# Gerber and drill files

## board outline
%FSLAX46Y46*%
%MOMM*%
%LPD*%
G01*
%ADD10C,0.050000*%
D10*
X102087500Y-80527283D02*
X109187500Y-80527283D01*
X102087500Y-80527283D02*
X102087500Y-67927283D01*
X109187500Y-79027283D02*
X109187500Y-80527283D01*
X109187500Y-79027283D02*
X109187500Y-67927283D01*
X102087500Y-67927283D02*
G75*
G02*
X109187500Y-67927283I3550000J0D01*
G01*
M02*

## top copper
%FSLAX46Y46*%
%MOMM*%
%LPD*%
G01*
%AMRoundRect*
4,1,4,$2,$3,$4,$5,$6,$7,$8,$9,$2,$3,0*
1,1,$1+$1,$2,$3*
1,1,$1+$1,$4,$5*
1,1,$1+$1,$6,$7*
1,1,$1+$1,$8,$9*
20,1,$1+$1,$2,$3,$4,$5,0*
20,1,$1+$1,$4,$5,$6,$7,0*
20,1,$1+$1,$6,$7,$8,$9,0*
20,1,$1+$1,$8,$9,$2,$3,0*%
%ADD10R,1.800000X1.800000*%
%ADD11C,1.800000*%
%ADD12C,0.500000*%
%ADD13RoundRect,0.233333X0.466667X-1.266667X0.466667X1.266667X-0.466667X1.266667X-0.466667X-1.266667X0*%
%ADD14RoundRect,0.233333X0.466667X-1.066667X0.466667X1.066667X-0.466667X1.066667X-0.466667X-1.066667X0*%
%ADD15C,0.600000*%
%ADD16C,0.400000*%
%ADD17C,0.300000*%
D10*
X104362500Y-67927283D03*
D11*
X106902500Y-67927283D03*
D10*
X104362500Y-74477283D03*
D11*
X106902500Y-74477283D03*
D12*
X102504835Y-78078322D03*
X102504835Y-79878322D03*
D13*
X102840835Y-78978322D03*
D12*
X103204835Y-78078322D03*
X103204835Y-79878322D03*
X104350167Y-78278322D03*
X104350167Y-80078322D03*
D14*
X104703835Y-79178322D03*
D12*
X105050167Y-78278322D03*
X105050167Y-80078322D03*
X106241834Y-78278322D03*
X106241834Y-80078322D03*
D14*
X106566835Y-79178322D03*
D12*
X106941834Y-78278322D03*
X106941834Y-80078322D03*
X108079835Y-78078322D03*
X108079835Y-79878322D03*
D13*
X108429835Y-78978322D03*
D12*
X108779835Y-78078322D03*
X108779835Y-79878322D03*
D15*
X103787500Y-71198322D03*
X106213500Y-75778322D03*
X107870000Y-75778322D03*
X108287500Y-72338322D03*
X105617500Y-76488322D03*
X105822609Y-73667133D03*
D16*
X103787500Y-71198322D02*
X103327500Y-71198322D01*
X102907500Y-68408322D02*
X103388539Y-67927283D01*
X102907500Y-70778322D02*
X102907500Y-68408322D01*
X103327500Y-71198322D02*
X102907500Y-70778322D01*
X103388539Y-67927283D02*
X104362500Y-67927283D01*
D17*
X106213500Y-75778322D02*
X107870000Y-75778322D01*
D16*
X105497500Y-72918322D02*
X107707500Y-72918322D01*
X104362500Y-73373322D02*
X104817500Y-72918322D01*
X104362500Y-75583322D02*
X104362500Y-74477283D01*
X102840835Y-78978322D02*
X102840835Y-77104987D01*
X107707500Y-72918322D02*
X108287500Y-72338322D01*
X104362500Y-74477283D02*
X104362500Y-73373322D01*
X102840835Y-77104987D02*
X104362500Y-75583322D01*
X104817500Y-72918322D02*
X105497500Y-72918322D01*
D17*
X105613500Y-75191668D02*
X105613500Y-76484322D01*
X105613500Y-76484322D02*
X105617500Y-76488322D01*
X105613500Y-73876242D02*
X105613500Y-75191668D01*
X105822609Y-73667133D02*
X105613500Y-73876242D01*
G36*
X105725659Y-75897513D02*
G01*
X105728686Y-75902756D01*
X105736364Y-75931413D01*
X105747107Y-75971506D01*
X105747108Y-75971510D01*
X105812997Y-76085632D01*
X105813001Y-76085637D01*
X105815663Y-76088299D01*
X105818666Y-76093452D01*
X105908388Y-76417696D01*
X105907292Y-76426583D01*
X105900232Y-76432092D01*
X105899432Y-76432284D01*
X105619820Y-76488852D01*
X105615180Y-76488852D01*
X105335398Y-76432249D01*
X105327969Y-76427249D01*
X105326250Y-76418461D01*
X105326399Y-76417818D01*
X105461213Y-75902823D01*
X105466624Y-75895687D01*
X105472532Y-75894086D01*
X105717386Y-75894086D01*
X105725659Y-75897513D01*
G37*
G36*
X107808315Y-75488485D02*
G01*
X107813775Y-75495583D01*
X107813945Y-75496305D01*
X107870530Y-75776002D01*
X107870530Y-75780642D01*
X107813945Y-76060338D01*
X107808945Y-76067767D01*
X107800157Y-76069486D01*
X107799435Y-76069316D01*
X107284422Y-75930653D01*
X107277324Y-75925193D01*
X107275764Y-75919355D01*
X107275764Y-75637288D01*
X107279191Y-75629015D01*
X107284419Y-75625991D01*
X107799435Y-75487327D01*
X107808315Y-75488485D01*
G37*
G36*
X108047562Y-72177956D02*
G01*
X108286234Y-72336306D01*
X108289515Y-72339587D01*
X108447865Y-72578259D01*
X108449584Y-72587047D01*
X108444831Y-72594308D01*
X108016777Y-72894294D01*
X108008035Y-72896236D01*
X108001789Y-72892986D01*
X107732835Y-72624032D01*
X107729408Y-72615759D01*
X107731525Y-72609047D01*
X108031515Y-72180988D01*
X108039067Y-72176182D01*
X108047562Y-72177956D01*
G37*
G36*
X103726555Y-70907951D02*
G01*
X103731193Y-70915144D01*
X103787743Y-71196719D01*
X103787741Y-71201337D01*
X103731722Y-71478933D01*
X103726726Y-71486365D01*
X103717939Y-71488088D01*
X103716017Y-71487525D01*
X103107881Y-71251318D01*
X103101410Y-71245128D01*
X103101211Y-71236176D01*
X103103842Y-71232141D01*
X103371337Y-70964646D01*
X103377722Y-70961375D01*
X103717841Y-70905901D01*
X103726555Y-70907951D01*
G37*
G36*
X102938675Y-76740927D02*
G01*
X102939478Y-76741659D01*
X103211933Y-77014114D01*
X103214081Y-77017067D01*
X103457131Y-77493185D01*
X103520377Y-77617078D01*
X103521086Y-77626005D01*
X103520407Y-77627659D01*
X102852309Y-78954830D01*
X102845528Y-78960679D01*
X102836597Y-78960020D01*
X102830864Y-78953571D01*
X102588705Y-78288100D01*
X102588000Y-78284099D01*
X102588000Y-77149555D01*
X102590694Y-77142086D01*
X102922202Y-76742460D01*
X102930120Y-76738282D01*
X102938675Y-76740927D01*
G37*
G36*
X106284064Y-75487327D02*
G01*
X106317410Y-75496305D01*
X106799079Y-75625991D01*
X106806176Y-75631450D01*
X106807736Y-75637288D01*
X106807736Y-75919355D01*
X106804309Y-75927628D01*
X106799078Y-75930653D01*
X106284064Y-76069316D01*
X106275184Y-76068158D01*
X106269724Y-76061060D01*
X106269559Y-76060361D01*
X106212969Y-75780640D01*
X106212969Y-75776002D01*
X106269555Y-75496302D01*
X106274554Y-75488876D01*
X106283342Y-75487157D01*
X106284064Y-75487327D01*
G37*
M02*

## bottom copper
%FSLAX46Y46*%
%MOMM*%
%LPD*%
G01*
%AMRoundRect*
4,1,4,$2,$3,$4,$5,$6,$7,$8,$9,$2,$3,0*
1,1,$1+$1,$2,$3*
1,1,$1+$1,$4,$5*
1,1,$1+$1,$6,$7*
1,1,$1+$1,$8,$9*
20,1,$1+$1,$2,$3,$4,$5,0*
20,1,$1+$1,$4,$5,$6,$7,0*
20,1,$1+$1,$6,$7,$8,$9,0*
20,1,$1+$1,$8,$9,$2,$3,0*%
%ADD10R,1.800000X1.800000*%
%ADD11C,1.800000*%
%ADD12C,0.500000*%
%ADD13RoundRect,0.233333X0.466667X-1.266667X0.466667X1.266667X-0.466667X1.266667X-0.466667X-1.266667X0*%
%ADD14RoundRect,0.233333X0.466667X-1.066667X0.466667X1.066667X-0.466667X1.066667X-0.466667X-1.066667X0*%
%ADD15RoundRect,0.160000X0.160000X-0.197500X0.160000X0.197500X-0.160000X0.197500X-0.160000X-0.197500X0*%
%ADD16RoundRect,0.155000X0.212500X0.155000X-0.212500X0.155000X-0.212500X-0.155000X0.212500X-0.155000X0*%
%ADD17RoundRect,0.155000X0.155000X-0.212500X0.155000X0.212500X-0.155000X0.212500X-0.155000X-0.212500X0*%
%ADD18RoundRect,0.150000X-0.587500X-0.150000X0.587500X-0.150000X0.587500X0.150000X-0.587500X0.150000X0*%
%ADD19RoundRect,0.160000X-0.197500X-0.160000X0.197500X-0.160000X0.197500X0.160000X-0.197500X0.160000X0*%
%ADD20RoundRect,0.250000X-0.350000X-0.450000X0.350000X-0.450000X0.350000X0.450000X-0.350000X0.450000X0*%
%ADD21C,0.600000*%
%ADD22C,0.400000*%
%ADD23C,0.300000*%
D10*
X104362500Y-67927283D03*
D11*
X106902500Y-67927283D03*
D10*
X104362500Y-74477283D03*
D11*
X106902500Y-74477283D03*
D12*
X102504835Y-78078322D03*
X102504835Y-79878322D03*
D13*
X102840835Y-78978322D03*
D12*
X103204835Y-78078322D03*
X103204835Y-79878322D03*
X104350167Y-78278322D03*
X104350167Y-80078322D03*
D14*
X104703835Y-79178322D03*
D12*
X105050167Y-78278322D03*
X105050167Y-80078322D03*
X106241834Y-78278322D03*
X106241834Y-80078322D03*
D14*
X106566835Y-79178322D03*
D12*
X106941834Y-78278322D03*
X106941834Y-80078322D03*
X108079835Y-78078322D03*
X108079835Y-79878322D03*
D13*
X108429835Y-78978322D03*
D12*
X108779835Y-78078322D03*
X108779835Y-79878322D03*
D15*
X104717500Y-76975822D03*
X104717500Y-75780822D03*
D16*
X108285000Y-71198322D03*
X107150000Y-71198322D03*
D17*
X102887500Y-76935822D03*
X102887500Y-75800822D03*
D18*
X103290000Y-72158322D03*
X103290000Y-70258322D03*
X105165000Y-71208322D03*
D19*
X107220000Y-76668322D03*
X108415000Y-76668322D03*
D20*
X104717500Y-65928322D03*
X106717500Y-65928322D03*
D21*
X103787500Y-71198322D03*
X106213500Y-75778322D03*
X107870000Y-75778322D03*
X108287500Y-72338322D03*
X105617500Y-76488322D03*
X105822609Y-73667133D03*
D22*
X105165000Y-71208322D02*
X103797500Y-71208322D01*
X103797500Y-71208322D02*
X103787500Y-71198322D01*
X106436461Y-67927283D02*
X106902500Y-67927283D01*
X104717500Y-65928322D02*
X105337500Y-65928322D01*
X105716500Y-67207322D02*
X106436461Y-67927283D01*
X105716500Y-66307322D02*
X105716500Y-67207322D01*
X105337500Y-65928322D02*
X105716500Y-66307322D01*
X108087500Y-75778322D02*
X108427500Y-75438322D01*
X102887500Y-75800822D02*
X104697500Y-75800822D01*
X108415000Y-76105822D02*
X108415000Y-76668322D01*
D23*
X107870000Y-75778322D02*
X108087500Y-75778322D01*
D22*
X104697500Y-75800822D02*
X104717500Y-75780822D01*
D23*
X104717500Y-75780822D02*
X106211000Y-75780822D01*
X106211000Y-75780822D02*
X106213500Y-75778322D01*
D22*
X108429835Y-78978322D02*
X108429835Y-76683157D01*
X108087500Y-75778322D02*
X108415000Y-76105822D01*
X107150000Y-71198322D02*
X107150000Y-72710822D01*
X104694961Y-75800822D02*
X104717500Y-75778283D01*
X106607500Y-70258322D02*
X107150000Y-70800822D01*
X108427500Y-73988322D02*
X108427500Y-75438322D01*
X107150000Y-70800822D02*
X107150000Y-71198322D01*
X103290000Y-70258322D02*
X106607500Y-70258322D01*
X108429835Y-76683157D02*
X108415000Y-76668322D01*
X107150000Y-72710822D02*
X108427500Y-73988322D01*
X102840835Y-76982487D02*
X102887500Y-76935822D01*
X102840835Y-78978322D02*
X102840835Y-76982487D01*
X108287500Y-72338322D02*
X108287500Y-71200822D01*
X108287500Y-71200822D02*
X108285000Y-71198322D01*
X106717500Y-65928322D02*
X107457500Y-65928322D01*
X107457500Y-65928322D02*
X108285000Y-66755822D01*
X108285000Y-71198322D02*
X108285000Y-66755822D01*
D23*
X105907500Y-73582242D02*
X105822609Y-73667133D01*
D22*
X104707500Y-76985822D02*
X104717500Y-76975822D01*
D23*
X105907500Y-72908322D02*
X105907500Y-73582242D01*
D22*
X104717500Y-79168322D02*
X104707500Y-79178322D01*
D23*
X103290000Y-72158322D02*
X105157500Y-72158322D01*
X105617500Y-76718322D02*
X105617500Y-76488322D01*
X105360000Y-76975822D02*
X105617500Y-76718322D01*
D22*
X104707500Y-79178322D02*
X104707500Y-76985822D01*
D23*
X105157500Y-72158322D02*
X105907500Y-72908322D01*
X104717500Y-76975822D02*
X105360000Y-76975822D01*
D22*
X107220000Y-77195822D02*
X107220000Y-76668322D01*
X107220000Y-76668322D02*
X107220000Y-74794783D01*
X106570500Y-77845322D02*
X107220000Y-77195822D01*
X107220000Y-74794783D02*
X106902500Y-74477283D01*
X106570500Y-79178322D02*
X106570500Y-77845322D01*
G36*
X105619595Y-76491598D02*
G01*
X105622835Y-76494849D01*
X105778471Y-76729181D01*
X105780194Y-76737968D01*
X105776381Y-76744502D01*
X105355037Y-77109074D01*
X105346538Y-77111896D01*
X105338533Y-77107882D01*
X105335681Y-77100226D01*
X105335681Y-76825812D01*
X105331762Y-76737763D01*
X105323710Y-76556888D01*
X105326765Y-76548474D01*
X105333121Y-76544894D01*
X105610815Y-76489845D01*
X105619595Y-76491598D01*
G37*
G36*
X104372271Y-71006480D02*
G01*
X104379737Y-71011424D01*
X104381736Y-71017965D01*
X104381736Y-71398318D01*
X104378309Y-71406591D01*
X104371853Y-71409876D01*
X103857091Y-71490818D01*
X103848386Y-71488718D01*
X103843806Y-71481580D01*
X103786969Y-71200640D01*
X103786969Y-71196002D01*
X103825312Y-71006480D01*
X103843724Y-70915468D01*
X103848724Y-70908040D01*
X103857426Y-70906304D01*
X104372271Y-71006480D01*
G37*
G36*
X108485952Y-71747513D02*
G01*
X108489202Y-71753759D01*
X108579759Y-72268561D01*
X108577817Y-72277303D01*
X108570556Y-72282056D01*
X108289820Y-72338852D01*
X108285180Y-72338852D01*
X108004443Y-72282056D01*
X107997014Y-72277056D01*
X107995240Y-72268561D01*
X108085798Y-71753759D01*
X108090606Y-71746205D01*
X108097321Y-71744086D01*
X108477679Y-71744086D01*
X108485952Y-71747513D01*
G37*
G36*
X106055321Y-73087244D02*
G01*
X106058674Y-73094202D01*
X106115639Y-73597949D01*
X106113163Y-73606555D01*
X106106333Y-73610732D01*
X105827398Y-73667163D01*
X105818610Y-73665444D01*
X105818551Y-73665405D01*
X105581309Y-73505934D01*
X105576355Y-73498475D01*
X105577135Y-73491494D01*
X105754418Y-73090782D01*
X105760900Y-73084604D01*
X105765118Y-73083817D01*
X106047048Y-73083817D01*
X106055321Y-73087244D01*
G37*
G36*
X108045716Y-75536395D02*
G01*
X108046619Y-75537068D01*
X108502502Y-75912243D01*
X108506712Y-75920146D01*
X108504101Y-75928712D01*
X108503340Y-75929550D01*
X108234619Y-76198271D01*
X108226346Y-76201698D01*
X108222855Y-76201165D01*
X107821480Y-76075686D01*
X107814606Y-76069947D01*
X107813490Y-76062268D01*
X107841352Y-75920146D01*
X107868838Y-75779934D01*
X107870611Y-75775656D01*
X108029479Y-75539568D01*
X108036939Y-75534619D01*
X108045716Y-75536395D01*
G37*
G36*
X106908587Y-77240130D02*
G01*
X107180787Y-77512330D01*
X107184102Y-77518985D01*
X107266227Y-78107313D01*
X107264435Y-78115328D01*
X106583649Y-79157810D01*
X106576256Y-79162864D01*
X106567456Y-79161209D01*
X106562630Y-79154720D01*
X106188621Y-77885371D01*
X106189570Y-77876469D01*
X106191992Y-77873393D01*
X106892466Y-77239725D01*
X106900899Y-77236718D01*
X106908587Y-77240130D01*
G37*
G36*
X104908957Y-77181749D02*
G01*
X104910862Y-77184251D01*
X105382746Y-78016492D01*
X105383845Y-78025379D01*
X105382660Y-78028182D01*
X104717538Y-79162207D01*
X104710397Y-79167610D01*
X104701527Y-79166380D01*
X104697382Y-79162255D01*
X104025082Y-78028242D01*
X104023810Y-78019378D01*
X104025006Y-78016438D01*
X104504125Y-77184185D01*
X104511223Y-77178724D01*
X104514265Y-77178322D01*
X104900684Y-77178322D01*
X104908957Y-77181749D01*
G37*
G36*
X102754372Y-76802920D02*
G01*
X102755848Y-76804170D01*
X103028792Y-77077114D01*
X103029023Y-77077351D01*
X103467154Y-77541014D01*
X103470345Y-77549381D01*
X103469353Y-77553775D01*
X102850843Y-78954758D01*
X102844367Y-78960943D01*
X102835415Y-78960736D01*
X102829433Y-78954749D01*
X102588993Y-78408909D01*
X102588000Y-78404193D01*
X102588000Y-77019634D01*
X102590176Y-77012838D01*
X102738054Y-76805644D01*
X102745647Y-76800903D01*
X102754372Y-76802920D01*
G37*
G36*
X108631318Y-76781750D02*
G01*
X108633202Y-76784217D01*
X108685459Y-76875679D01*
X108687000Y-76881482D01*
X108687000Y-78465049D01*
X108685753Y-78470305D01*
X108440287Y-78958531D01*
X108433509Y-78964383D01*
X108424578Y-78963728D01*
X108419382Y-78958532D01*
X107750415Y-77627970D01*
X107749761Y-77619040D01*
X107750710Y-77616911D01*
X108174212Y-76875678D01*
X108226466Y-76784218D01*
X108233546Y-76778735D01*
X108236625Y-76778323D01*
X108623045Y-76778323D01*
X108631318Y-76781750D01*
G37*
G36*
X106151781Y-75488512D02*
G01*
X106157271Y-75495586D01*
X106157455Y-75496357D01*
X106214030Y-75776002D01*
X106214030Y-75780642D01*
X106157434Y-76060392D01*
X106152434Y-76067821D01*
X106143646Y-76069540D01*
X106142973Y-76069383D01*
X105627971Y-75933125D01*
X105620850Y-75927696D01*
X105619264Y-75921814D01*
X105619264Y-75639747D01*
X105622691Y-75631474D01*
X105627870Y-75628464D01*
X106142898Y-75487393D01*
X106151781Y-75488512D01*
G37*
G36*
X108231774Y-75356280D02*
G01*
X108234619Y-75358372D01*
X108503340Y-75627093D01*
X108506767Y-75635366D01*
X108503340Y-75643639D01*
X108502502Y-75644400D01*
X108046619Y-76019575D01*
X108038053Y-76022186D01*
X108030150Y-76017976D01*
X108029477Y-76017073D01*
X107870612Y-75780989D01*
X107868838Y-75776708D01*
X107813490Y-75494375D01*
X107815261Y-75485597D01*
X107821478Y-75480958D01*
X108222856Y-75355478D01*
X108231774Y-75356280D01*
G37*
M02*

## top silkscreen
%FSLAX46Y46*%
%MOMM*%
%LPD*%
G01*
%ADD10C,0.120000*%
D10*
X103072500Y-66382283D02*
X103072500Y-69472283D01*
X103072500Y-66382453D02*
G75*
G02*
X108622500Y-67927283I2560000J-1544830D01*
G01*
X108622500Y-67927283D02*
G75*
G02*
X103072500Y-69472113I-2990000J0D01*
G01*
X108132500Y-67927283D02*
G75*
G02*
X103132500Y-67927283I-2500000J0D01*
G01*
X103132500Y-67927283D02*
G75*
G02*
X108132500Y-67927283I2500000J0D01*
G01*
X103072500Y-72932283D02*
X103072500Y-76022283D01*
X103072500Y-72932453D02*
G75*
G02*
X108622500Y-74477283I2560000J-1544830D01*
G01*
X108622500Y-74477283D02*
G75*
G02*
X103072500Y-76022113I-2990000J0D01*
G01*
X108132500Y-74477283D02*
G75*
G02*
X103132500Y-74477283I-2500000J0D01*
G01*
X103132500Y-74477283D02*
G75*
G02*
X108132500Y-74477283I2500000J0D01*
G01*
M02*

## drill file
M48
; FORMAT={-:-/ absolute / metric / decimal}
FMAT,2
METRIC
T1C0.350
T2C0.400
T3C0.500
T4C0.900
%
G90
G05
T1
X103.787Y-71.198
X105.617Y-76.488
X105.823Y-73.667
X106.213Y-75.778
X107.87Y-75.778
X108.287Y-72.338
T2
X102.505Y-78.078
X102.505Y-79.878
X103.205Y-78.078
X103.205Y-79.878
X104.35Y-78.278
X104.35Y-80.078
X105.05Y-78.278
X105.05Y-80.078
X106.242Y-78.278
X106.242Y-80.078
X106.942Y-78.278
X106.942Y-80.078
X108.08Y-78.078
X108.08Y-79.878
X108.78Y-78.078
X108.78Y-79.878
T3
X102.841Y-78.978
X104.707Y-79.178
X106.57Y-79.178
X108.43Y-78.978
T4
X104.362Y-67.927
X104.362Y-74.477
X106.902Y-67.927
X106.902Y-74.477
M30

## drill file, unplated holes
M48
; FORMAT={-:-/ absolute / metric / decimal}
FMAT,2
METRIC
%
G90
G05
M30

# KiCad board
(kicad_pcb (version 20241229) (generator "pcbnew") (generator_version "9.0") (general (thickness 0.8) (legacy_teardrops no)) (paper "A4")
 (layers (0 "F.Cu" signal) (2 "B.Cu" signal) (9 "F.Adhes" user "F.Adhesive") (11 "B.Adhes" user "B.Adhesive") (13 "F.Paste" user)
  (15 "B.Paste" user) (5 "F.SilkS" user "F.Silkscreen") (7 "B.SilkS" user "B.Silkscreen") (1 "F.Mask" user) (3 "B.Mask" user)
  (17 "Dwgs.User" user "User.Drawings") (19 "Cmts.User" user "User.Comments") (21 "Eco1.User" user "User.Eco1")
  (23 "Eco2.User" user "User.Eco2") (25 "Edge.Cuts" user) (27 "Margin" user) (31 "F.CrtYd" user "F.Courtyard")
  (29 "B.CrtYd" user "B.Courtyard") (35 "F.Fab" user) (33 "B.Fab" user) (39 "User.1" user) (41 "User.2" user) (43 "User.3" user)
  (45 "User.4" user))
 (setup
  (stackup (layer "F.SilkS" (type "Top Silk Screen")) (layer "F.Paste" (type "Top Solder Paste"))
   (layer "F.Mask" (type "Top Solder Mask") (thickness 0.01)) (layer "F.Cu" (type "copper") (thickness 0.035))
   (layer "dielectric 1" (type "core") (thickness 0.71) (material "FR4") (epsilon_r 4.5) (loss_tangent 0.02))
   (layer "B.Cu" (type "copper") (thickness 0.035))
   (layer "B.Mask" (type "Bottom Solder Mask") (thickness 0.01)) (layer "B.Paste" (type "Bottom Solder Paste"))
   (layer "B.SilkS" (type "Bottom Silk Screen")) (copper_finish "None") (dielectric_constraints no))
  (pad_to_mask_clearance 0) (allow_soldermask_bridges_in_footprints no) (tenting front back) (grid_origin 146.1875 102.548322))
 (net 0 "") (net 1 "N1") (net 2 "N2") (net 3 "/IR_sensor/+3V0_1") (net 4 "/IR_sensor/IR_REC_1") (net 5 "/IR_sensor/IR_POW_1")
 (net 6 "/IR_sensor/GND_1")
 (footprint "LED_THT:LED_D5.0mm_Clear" (layer "F.Cu") (at 104.3625 67.927283)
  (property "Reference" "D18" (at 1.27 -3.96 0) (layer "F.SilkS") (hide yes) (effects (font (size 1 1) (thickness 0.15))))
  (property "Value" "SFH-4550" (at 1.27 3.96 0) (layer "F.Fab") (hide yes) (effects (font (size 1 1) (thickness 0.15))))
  (fp_line (start -1.29 -1.545) (end -1.29 1.545) (stroke (width 0.12) (type solid)) (layer "F.SilkS"))
  (fp_arc (start -1.29 -1.54483) (mid 2.071779 -2.880495) (end 4.26 0) (stroke (width 0.12) (type solid)) (layer "F.SilkS"))
  (fp_arc (start 4.26 0) (mid 2.071779 2.880495) (end -1.29 1.54483) (stroke (width 0.12) (type solid)) (layer "F.SilkS"))
  (fp_circle (center 1.27 0) (end 3.77 0) (stroke (width 0.12) (type solid)) (fill no) (layer "F.SilkS"))
  (pad "1" thru_hole rect (at 0 0) (size 1.8 1.8) (drill 0.9) (layers "*.Cu" "*.Mask") (remove_unused_layers no) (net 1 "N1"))
  (pad "2" thru_hole circle (at 2.54 0) (size 1.8 1.8) (drill 0.9) (layers "*.Cu" "*.Mask") (remove_unused_layers no) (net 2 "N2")))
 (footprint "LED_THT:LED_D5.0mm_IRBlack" (layer "F.Cu") (at 104.3625 74.477283)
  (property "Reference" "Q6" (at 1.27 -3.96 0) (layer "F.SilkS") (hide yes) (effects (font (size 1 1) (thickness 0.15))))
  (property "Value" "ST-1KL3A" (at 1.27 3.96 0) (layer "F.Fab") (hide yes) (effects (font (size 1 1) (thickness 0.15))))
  (fp_line (start -1.29 -1.545) (end -1.29 1.545) (stroke (width 0.12) (type solid)) (layer "F.SilkS"))
  (fp_arc (start -1.29 -1.54483) (mid 2.071779 -2.880495) (end 4.26 0) (stroke (width 0.12) (type solid)) (layer "F.SilkS"))
  (fp_arc (start 4.26 0) (mid 2.071779 2.880495) (end -1.29 1.54483) (stroke (width 0.12) (type solid)) (layer "F.SilkS"))
  (fp_circle (center 1.27 0) (end 3.77 0) (stroke (width 0.12) (type solid)) (fill no) (layer "F.SilkS"))
  (pad "1" thru_hole rect (at 0 0) (size 1.8 1.8) (drill 0.9) (layers "*.Cu" "*.Mask") (remove_unused_layers no) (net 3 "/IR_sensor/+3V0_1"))
  (pad "2" thru_hole circle (at 2.54 0) (size 1.8 1.8) (drill 0.9) (layers "*.Cu" "*.Mask") (remove_unused_layers no)
   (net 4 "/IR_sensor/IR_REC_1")))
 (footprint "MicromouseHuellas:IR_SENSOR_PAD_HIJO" (layer "F.Cu") (at 105.6375 79.178322)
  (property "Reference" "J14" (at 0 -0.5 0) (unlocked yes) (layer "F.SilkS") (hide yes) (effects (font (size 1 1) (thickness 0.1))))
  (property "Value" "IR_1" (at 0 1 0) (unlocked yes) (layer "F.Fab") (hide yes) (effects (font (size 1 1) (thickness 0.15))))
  (pad "1" thru_hole circle (at -3.132665 -1.1 90) (size 0.5 0.5) (drill 0.4) (layers "*.Cu" "*.Mask") (remove_unused_layers no)
   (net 3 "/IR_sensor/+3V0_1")
   (teardrops (best_length_ratio 0.5) (max_length 1) (best_width_ratio 1) (max_width 2) (curved_edges no) (filter_ratio 0.9) (enabled yes)
    (allow_two_segments yes) (prefer_zone_connections yes)))
  (pad "1" thru_hole circle (at -3.132665 0.7 90) (size 0.5 0.5) (drill 0.4) (layers "*.Cu" "*.Mask") (remove_unused_layers no)
   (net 3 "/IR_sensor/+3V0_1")
   (teardrops (best_length_ratio 0.5) (max_length 1) (best_width_ratio 1) (max_width 2) (curved_edges no) (filter_ratio 0.9) (enabled yes)
    (allow_two_segments yes) (prefer_zone_connections yes)))
  (pad "1" thru_hole roundrect (at -2.796665 -0.2 90) (size 3 1.4) (drill 0.5) (layers "*.Cu" "*.Mask") (remove_unused_layers no)
   (roundrect_rratio 0.1666666667) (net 3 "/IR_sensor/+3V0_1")
   (teardrops (best_length_ratio 0.5) (max_length 1) (best_width_ratio 1) (max_width 2) (curved_edges no) (filter_ratio 0.9) (enabled yes)
    (allow_two_segments yes) (prefer_zone_connections yes)))
  (pad "1" thru_hole circle (at -2.432665 -1.1 90) (size 0.5 0.5) (drill 0.4) (layers "*.Cu" "*.Mask") (remove_unused_layers no)
   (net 3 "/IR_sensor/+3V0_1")
   (teardrops (best_length_ratio 0.5) (max_length 1) (best_width_ratio 1) (max_width 2) (curved_edges no) (filter_ratio 0.9) (enabled yes)
    (allow_two_segments yes) (prefer_zone_connections yes)))
  (pad "1" thru_hole circle (at -2.432665 0.7 90) (size 0.5 0.5) (drill 0.4) (layers "*.Cu" "*.Mask") (remove_unused_layers no)
   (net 3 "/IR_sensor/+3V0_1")
   (teardrops (best_length_ratio 0.5) (max_length 1) (best_width_ratio 1) (max_width 2) (curved_edges no) (filter_ratio 0.9) (enabled yes)
    (allow_two_segments yes) (prefer_zone_connections yes)))
  (pad "2" thru_hole circle (at -1.287333 -0.9 90) (size 0.5 0.5) (drill 0.4) (layers "*.Cu" "*.Mask") (remove_unused_layers no)
   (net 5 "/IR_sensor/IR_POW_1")
   (teardrops (best_length_ratio 0.5) (max_length 1) (best_width_ratio 1) (max_width 2) (curved_edges no) (filter_ratio 0.9) (enabled yes)
    (allow_two_segments yes) (prefer_zone_connections yes)))
  (pad "2" thru_hole circle (at -1.287333 0.9 90) (size 0.5 0.5) (drill 0.4) (layers "*.Cu" "*.Mask") (remove_unused_layers no)
   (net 5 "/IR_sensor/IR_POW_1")
   (teardrops (best_length_ratio 0.5) (max_length 1) (best_width_ratio 1) (max_width 2) (curved_edges no) (filter_ratio 0.9) (enabled yes)
    (allow_two_segments yes) (prefer_zone_connections yes)))
  (pad "2" thru_hole roundrect (at -0.93 0 90) (size 2.6 1.4) (drill 0.5 (offset 0 -0.003665)) (layers "*.Cu" "*.Mask")
   (remove_unused_layers no) (roundrect_rratio 0.1666666667) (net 5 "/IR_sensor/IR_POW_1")
   (teardrops (best_length_ratio 0.5) (max_length 1) (best_width_ratio 1) (max_width 2) (curved_edges no) (filter_ratio 0.9) (enabled yes)
    (allow_two_segments yes) (prefer_zone_connections yes)))
  (pad "2" thru_hole circle (at -0.587333 -0.9 90) (size 0.5 0.5) (drill 0.4) (layers "*.Cu" "*.Mask") (remove_unused_layers no)
   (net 5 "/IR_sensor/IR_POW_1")
   (teardrops (best_length_ratio 0.5) (max_length 1) (best_width_ratio 1) (max_width 2) (curved_edges no) (filter_ratio 0.9) (enabled yes)
    (allow_two_segments yes) (prefer_zone_connections yes)))
  (pad "2" thru_hole circle (at -0.587333 0.9 90) (size 0.5 0.5) (drill 0.4) (layers "*.Cu" "*.Mask") (remove_unused_layers no)
   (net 5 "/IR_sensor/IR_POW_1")
   (teardrops (best_length_ratio 0.5) (max_length 1) (best_width_ratio 1) (max_width 2) (curved_edges no) (filter_ratio 0.9) (enabled yes)
    (allow_two_segments yes) (prefer_zone_connections yes)))
  (pad "3" thru_hole circle (at 0.604334 -0.9 90) (size 0.5 0.5) (drill 0.4) (layers "*.Cu" "*.Mask") (remove_unused_layers no)
   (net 4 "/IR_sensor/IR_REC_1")
   (teardrops (best_length_ratio 0.5) (max_length 1) (best_width_ratio 1) (max_width 2) (curved_edges no) (filter_ratio 0.9) (enabled yes)
    (allow_two_segments yes) (prefer_zone_connections yes)))
  (pad "3" thru_hole circle (at 0.604334 0.9 90) (size 0.5 0.5) (drill 0.4) (layers "*.Cu" "*.Mask") (remove_unused_layers no)
   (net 4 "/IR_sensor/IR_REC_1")
   (teardrops (best_length_ratio 0.5) (max_length 1) (best_width_ratio 1) (max_width 2) (curved_edges no) (filter_ratio 0.9) (enabled yes)
    (allow_two_segments yes) (prefer_zone_connections yes)))
  (pad "3" thru_hole roundrect (at 0.933 0 90) (size 2.6 1.4) (drill 0.5 (offset 0 -0.003665)) (layers "*.Cu" "*.Mask")
   (remove_unused_layers no) (roundrect_rratio 0.1666666667) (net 4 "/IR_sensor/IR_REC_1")
   (teardrops (best_length_ratio 0.5) (max_length 1) (best_width_ratio 1) (max_width 2) (curved_edges no) (filter_ratio 0.9) (enabled yes)
    (allow_two_segments yes) (prefer_zone_connections yes)))
  (pad "3" thru_hole circle (at 1.304334 -0.9 90) (size 0.5 0.5) (drill 0.4) (layers "*.Cu" "*.Mask") (remove_unused_layers no)
   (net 4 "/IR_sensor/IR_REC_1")
   (teardrops (best_length_ratio 0.5) (max_length 1) (best_width_ratio 1) (max_width 2) (curved_edges no) (filter_ratio 0.9) (enabled yes)
    (allow_two_segments yes) (prefer_zone_connections yes)))
  (pad "3" thru_hole circle (at 1.304334 0.9 90) (size 0.5 0.5) (drill 0.4) (layers "*.Cu" "*.Mask") (remove_unused_layers no)
   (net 4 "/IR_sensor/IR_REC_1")
   (teardrops (best_length_ratio 0.5) (max_length 1) (best_width_ratio 1) (max_width 2) (curved_edges no) (filter_ratio 0.9) (enabled yes)
    (allow_two_segments yes) (prefer_zone_connections yes)))
  (pad "4" thru_hole circle (at 2.442335 -1.1 90) (size 0.5 0.5) (drill 0.4) (layers "*.Cu" "*.Mask") (remove_unused_layers no)
   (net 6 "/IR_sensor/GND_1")
   (teardrops (best_length_ratio 0.5) (max_length 1) (best_width_ratio 1) (max_width 2) (curved_edges no) (filter_ratio 0.9) (enabled yes)
    (allow_two_segments yes) (prefer_zone_connections yes)))
  (pad "4" thru_hole circle (at 2.442335 0.7 90) (size 0.5 0.5) (drill 0.4) (layers "*.Cu" "*.Mask") (remove_unused_layers no)
   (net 6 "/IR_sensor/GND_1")
   (teardrops (best_length_ratio 0.5) (max_length 1) (best_width_ratio 1) (max_width 2) (curved_edges no) (filter_ratio 0.9) (enabled yes)
    (allow_two_segments yes) (prefer_zone_connections yes)))
  (pad "4" thru_hole roundrect (at 2.792335 -0.2 90) (size 3 1.4) (drill 0.5) (layers "*.Cu" "*.Mask") (remove_unused_layers no)
   (roundrect_rratio 0.1666666667) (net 6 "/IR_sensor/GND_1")
   (teardrops (best_length_ratio 0.5) (max_length 1) (best_width_ratio 1) (max_width 2) (curved_edges no) (filter_ratio 0.9) (enabled yes)
    (allow_two_segments yes) (prefer_zone_connections yes)))
  (pad "4" thru_hole circle (at 3.142335 -1.1 90) (size 0.5 0.5) (drill 0.4) (layers "*.Cu" "*.Mask") (remove_unused_layers no)
   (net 6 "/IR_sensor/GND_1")
   (teardrops (best_length_ratio 0.5) (max_length 1) (best_width_ratio 1) (max_width 2) (curved_edges no) (filter_ratio 0.9) (enabled yes)
    (allow_two_segments yes) (prefer_zone_connections yes)))
  (pad "4" thru_hole circle (at 3.142335 0.7 90) (size 0.5 0.5) (drill 0.4) (layers "*.Cu" "*.Mask") (remove_unused_layers no)
   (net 6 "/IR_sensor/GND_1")
   (teardrops (best_length_ratio 0.5) (max_length 1) (best_width_ratio 1) (max_width 2) (curved_edges no) (filter_ratio 0.9) (enabled yes)
    (allow_two_segments yes) (prefer_zone_connections yes))))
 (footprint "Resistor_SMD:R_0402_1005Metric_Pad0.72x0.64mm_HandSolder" (layer "B.Cu") (at 104.7175 76.378322 90)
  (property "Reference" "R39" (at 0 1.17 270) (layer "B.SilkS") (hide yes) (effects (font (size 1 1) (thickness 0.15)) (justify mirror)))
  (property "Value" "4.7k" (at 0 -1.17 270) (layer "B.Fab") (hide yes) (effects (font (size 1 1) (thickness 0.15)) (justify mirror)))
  (pad "1" smd roundrect (at -0.5975 0 90) (size 0.715 0.64) (layers "B.Cu" "B.Mask" "B.Paste") (roundrect_rratio 0.25)
   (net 5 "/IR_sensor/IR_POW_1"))
  (pad "2" smd roundrect (at 0.5975 0 90) (size 0.715 0.64) (layers "B.Cu" "B.Mask" "B.Paste") (roundrect_rratio 0.25)
   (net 6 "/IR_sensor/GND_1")))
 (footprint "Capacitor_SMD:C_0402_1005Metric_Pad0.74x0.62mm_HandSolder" (layer "B.Cu") (at 107.7175 71.198322 180)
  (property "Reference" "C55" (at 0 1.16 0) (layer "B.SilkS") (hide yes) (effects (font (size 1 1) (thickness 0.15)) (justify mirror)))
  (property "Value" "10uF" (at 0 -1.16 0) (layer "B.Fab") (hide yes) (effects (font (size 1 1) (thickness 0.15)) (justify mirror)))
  (pad "1" smd roundrect (at -0.5675 0 180) (size 0.735 0.62) (layers "B.Cu" "B.Mask" "B.Paste") (roundrect_rratio 0.25)
   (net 3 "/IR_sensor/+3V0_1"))
  (pad "2" smd roundrect (at 0.5675 0 180) (size 0.735 0.62) (layers "B.Cu" "B.Mask" "B.Paste") (roundrect_rratio 0.25)
   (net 6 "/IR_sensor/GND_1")))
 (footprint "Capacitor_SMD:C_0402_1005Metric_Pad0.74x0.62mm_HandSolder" (layer "B.Cu") (at 102.8875 76.368322 90)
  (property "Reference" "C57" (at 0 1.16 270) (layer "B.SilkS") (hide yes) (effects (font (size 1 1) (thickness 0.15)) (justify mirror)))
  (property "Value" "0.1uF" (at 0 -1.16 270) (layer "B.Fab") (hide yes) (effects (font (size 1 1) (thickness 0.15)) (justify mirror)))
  (pad "1" smd roundrect (at -0.5675 0 90) (size 0.735 0.62) (layers "B.Cu" "B.Mask" "B.Paste") (roundrect_rratio 0.25)
   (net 3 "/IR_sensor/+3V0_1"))
  (pad "2" smd roundrect (at 0.5675 0 90) (size 0.735 0.62) (layers "B.Cu" "B.Mask" "B.Paste") (roundrect_rratio 0.25)
   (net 6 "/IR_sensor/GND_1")))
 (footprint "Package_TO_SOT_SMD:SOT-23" (layer "B.Cu") (at 104.2275 71.208322)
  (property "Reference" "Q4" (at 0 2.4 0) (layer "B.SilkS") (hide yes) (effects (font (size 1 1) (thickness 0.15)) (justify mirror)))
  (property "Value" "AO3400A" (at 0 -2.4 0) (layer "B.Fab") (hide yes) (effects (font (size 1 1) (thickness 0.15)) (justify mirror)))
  (pad "1" smd roundrect (at -0.9375 0.95) (size 1.475 0.6) (layers "B.Cu" "B.Mask" "B.Paste") (roundrect_rratio 0.25)
   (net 5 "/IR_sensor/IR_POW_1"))
  (pad "2" smd roundrect (at -0.9375 -0.95) (size 1.475 0.6) (layers "B.Cu" "B.Mask" "B.Paste") (roundrect_rratio 0.25)
   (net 6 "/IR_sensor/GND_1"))
  (pad "3" smd roundrect (at 0.9375 0) (size 1.475 0.6) (layers "B.Cu" "B.Mask" "B.Paste") (roundrect_rratio 0.25) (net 1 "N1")))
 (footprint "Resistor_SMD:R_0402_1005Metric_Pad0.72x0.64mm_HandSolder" (layer "B.Cu") (at 107.8175 76.668322)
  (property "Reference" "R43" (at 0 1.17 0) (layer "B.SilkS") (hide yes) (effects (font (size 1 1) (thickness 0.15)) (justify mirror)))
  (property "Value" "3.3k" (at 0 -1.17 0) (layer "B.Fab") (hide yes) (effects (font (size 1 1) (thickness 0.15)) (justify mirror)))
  (pad "1" smd roundrect (at -0.5975 0) (size 0.715 0.64) (layers "B.Cu" "B.Mask" "B.Paste") (roundrect_rratio 0.25)
   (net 4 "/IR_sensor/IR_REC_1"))
  (pad "2" smd roundrect (at 0.5975 0) (size 0.715 0.64) (layers "B.Cu" "B.Mask" "B.Paste") (roundrect_rratio 0.25)
   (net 6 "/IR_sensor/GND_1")))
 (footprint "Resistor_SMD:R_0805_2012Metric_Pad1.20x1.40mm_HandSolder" (layer "B.Cu") (at 105.7175 65.928322)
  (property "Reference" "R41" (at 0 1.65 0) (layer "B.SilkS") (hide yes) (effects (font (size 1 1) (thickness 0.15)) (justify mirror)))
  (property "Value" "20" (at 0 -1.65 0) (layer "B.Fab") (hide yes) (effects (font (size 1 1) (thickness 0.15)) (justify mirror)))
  (pad "1" smd roundrect (at -1 0) (size 1.2 1.4) (layers "B.Cu" "B.Mask" "B.Paste") (roundrect_rratio 0.208333) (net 2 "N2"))
  (pad "2" smd roundrect (at 1 0) (size 1.2 1.4) (layers "B.Cu" "B.Mask" "B.Paste") (roundrect_rratio 0.208333) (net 3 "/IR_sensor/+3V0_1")))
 (gr_line (start 102.0875 80.527283) (end 109.1875 80.527283) (stroke (width 0.05) (type solid)) (layer "Edge.Cuts"))
 (gr_line (start 102.0875 80.527283) (end 102.0875 67.927283) (stroke (width 0.05) (type solid)) (layer "Edge.Cuts"))
 (gr_line (start 109.1875 79.027283) (end 109.1875 80.527283) (stroke (width 0.05) (type default)) (layer "Edge.Cuts"))
 (gr_line (start 109.1875 79.027283) (end 109.1875 67.927283) (stroke (width 0.05) (type solid)) (layer "Edge.Cuts"))
 (gr_arc (start 102.0875 67.927283) (mid 105.6375 64.377283) (end 109.1875 67.927283) (stroke (width 0.05) (type default))
  (layer "Edge.Cuts"))
 (segment (start 103.7875 71.198322) (end 103.3275 71.198322) (width 0.4) (layer "F.Cu") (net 1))
 (segment (start 102.9075 68.408322) (end 103.388539 67.927283) (width 0.4) (layer "F.Cu") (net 1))
 (segment (start 102.9075 70.778322) (end 102.9075 68.408322) (width 0.4) (layer "F.Cu") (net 1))
 (segment (start 103.3275 71.198322) (end 102.9075 70.778322) (width 0.4) (layer "F.Cu") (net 1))
 (segment (start 103.388539 67.927283) (end 104.3625 67.927283) (width 0.4) (layer "F.Cu") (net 1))
 (via (at 103.7875 71.198322) (size 0.6) (drill 0.35) (layers "F.Cu" "B.Cu")
  (teardrops (best_length_ratio 0.5) (max_length 1) (best_width_ratio 1) (max_width 2) (curved_edges no) (filter_ratio 0.9) (enabled yes)
   (allow_two_segments yes) (prefer_zone_connections yes))
  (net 1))
 (segment (start 105.165 71.208322) (end 103.7975 71.208322) (width 0.4) (layer "B.Cu") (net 1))
 (segment (start 103.7975 71.208322) (end 103.7875 71.198322) (width 0.4) (layer "B.Cu") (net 1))
 (segment (start 106.436461 67.927283) (end 106.9025 67.927283) (width 0.4) (layer "B.Cu") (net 2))
 (segment (start 104.7175 65.928322) (end 105.3375 65.928322) (width 0.4) (layer "B.Cu") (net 2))
 (segment (start 105.7165 67.207322) (end 106.436461 67.927283) (width 0.4) (layer "B.Cu") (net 2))
 (segment (start 105.7165 66.307322) (end 105.7165 67.207322) (width 0.4) (layer "B.Cu") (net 2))
 (segment (start 105.3375 65.928322) (end 105.7165 66.307322) (width 0.4) (layer "B.Cu") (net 2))
 (segment (start 106.2135 75.778322) (end 107.87 75.778322) (width 0.3) (layer "F.Cu") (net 6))
 (via (at 106.2135 75.778322) (size 0.6) (drill 0.35) (layers "F.Cu" "B.Cu")
  (teardrops (best_length_ratio 0.5) (max_length 1) (best_width_ratio 1) (max_width 2) (curved_edges no) (filter_ratio 0.9) (enabled yes)
   (allow_two_segments yes) (prefer_zone_connections yes))
  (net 6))
 (via (at 107.87 75.778322) (size 0.6) (drill 0.35) (layers "F.Cu" "B.Cu")
  (teardrops (best_length_ratio 0.5) (max_length 1) (best_width_ratio 1) (max_width 2) (curved_edges no) (filter_ratio 0.9) (enabled yes)
   (allow_two_segments yes) (prefer_zone_connections yes))
  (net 6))
 (segment (start 108.0875 75.778322) (end 108.4275 75.438322) (width 0.4) (layer "B.Cu") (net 6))
 (segment (start 102.8875 75.800822) (end 104.6975 75.800822) (width 0.4) (layer "B.Cu") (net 6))
 (segment (start 108.415 76.105822) (end 108.415 76.668322) (width 0.4) (layer "B.Cu") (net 6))
 (segment (start 107.87 75.778322) (end 108.0875 75.778322) (width 0.3) (layer "B.Cu") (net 6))
 (segment (start 104.6975 75.800822) (end 104.7175 75.780822) (width 0.4) (layer "B.Cu") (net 6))
 (segment (start 104.7175 75.780822) (end 106.211 75.780822) (width 0.3) (layer "B.Cu") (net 6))
 (segment (start 106.211 75.780822) (end 106.2135 75.778322) (width 0.3) (layer "B.Cu") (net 6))
 (segment (start 108.429835 78.978322) (end 108.429835 76.683157) (width 0.4) (layer "B.Cu") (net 6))
 (segment (start 108.0875 75.778322) (end 108.415 76.105822) (width 0.4) (layer "B.Cu") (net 6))
 (segment (start 107.15 71.198322) (end 107.15 72.710822) (width 0.4) (layer "B.Cu") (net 6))
 (segment (start 104.694961 75.800822) (end 104.7175 75.778283) (width 0.4) (layer "B.Cu") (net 6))
 (segment (start 106.6075 70.258322) (end 107.15 70.800822) (width 0.4) (layer "B.Cu") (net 6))
 (segment (start 108.4275 73.988322) (end 108.4275 75.438322) (width 0.4) (layer "B.Cu") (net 6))
 (segment (start 107.15 70.800822) (end 107.15 71.198322) (width 0.4) (layer "B.Cu") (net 6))
 (segment (start 103.29 70.258322) (end 106.6075 70.258322) (width 0.4) (layer "B.Cu") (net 6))
 (segment (start 108.429835 76.683157) (end 108.415 76.668322) (width 0.4) (layer "B.Cu") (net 6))
 (segment (start 107.15 72.710822) (end 108.4275 73.988322) (width 0.4) (layer "B.Cu") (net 6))
 (segment (start 105.4975 72.918322) (end 107.7075 72.918322) (width 0.4) (layer "F.Cu") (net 3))
 (segment (start 104.3625 73.373322) (end 104.8175 72.918322) (width 0.4) (layer "F.Cu") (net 3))
 (segment (start 104.3625 75.583322) (end 104.3625 74.477283) (width 0.4) (layer "F.Cu") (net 3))
 (segment (start 102.840835 78.978322) (end 102.840835 77.104987) (width 0.4) (layer "F.Cu") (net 3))
 (segment (start 107.7075 72.918322) (end 108.2875 72.338322) (width 0.4) (layer "F.Cu") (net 3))
 (segment (start 104.3625 74.477283) (end 104.3625 73.373322) (width 0.4) (layer "F.Cu") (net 3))
 (segment (start 102.840835 77.104987) (end 104.3625 75.583322) (width 0.4) (layer "F.Cu") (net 3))
 (segment (start 104.8175 72.918322) (end 105.4975 72.918322) (width 0.4) (layer "F.Cu") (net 3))
 (via (at 108.2875 72.338322) (size 0.6) (drill 0.35) (layers "F.Cu" "B.Cu")
  (teardrops (best_length_ratio 0.5) (max_length 1) (best_width_ratio 1) (max_width 2) (curved_edges no) (filter_ratio 0.9) (enabled yes)
   (allow_two_segments yes) (prefer_zone_connections yes))
  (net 3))
 (segment (start 102.840835 76.982487) (end 102.8875 76.935822) (width 0.4) (layer "B.Cu") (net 3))
 (segment (start 102.840835 78.978322) (end 102.840835 76.982487) (width 0.4) (layer "B.Cu") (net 3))
 (segment (start 108.2875 72.338322) (end 108.2875 71.200822) (width 0.4) (layer "B.Cu") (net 3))
 (segment (start 108.2875 71.200822) (end 108.285 71.198322) (width 0.4) (layer "B.Cu") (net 3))
 (segment (start 106.7175 65.928322) (end 107.4575 65.928322) (width 0.4) (layer "B.Cu") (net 3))
 (segment (start 107.4575 65.928322) (end 108.285 66.755822) (width 0.4) (layer "B.Cu") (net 3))
 (segment (start 108.285 71.198322) (end 108.285 66.755822) (width 0.4) (layer "B.Cu") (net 3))
 (segment (start 105.6135 75.191668) (end 105.6135 76.484322) (width 0.3) (layer "F.Cu") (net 5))
 (segment (start 105.6135 76.484322) (end 105.6175 76.488322) (width 0.3) (layer "F.Cu") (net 5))
 (segment (start 105.6135 73.876242) (end 105.6135 75.191668) (width 0.3) (layer "F.Cu") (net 5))
 (segment (start 105.822609 73.667133) (end 105.6135 73.876242) (width 0.3) (layer "F.Cu") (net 5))
 (via (at 105.6175 76.488322) (size 0.6) (drill 0.35) (layers "F.Cu" "B.Cu")
  (teardrops (best_length_ratio 0.5) (max_length 1) (best_width_ratio 1) (max_width 2) (curved_edges no) (filter_ratio 0.9) (enabled yes)
   (allow_two_segments yes) (prefer_zone_connections yes))
  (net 5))
 (via (at 105.822609 73.667133) (size 0.6) (drill 0.35) (layers "F.Cu" "B.Cu")
  (teardrops (best_length_ratio 0.5) (max_length 1) (best_width_ratio 1) (max_width 2) (curved_edges no) (filter_ratio 0.9) (enabled yes)
   (allow_two_segments yes) (prefer_zone_connections yes))
  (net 5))
 (segment (start 105.9075 73.582242) (end 105.822609 73.667133) (width 0.3) (layer "B.Cu") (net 5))
 (segment (start 104.7075 76.985822) (end 104.7175 76.975822) (width 0.4) (layer "B.Cu") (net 5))
 (segment (start 105.9075 72.908322) (end 105.9075 73.582242) (width 0.3) (layer "B.Cu") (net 5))
 (segment (start 104.7175 79.168322) (end 104.7075 79.178322) (width 0.4) (layer "B.Cu") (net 5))
 (segment (start 103.29 72.158322) (end 105.1575 72.158322) (width 0.3) (layer "B.Cu") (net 5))
 (segment (start 105.6175 76.718322) (end 105.6175 76.488322) (width 0.3) (layer "B.Cu") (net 5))
 (segment (start 105.36 76.975822) (end 105.6175 76.718322) (width 0.3) (layer "B.Cu") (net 5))
 (segment (start 104.7075 79.178322) (end 104.7075 76.985822) (width 0.4) (layer "B.Cu") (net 5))
 (segment (start 105.1575 72.158322) (end 105.9075 72.908322) (width 0.3) (layer "B.Cu") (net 5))
 (segment (start 104.7175 76.975822) (end 105.36 76.975822) (width 0.3) (layer "B.Cu") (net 5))
 (segment (start 107.22 77.195822) (end 107.22 76.668322) (width 0.4) (layer "B.Cu") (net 4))
 (segment (start 107.22 76.668322) (end 107.22 74.794783) (width 0.4) (layer "B.Cu") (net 4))
 (segment (start 106.5705 77.845322) (end 107.22 77.195822) (width 0.4) (layer "B.Cu") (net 4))
 (segment (start 107.22 74.794783) (end 106.9025 74.477283) (width 0.4) (layer "B.Cu") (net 4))
 (segment (start 106.5705 79.178322) (end 106.5705 77.845322) (width 0.4) (layer "B.Cu") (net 4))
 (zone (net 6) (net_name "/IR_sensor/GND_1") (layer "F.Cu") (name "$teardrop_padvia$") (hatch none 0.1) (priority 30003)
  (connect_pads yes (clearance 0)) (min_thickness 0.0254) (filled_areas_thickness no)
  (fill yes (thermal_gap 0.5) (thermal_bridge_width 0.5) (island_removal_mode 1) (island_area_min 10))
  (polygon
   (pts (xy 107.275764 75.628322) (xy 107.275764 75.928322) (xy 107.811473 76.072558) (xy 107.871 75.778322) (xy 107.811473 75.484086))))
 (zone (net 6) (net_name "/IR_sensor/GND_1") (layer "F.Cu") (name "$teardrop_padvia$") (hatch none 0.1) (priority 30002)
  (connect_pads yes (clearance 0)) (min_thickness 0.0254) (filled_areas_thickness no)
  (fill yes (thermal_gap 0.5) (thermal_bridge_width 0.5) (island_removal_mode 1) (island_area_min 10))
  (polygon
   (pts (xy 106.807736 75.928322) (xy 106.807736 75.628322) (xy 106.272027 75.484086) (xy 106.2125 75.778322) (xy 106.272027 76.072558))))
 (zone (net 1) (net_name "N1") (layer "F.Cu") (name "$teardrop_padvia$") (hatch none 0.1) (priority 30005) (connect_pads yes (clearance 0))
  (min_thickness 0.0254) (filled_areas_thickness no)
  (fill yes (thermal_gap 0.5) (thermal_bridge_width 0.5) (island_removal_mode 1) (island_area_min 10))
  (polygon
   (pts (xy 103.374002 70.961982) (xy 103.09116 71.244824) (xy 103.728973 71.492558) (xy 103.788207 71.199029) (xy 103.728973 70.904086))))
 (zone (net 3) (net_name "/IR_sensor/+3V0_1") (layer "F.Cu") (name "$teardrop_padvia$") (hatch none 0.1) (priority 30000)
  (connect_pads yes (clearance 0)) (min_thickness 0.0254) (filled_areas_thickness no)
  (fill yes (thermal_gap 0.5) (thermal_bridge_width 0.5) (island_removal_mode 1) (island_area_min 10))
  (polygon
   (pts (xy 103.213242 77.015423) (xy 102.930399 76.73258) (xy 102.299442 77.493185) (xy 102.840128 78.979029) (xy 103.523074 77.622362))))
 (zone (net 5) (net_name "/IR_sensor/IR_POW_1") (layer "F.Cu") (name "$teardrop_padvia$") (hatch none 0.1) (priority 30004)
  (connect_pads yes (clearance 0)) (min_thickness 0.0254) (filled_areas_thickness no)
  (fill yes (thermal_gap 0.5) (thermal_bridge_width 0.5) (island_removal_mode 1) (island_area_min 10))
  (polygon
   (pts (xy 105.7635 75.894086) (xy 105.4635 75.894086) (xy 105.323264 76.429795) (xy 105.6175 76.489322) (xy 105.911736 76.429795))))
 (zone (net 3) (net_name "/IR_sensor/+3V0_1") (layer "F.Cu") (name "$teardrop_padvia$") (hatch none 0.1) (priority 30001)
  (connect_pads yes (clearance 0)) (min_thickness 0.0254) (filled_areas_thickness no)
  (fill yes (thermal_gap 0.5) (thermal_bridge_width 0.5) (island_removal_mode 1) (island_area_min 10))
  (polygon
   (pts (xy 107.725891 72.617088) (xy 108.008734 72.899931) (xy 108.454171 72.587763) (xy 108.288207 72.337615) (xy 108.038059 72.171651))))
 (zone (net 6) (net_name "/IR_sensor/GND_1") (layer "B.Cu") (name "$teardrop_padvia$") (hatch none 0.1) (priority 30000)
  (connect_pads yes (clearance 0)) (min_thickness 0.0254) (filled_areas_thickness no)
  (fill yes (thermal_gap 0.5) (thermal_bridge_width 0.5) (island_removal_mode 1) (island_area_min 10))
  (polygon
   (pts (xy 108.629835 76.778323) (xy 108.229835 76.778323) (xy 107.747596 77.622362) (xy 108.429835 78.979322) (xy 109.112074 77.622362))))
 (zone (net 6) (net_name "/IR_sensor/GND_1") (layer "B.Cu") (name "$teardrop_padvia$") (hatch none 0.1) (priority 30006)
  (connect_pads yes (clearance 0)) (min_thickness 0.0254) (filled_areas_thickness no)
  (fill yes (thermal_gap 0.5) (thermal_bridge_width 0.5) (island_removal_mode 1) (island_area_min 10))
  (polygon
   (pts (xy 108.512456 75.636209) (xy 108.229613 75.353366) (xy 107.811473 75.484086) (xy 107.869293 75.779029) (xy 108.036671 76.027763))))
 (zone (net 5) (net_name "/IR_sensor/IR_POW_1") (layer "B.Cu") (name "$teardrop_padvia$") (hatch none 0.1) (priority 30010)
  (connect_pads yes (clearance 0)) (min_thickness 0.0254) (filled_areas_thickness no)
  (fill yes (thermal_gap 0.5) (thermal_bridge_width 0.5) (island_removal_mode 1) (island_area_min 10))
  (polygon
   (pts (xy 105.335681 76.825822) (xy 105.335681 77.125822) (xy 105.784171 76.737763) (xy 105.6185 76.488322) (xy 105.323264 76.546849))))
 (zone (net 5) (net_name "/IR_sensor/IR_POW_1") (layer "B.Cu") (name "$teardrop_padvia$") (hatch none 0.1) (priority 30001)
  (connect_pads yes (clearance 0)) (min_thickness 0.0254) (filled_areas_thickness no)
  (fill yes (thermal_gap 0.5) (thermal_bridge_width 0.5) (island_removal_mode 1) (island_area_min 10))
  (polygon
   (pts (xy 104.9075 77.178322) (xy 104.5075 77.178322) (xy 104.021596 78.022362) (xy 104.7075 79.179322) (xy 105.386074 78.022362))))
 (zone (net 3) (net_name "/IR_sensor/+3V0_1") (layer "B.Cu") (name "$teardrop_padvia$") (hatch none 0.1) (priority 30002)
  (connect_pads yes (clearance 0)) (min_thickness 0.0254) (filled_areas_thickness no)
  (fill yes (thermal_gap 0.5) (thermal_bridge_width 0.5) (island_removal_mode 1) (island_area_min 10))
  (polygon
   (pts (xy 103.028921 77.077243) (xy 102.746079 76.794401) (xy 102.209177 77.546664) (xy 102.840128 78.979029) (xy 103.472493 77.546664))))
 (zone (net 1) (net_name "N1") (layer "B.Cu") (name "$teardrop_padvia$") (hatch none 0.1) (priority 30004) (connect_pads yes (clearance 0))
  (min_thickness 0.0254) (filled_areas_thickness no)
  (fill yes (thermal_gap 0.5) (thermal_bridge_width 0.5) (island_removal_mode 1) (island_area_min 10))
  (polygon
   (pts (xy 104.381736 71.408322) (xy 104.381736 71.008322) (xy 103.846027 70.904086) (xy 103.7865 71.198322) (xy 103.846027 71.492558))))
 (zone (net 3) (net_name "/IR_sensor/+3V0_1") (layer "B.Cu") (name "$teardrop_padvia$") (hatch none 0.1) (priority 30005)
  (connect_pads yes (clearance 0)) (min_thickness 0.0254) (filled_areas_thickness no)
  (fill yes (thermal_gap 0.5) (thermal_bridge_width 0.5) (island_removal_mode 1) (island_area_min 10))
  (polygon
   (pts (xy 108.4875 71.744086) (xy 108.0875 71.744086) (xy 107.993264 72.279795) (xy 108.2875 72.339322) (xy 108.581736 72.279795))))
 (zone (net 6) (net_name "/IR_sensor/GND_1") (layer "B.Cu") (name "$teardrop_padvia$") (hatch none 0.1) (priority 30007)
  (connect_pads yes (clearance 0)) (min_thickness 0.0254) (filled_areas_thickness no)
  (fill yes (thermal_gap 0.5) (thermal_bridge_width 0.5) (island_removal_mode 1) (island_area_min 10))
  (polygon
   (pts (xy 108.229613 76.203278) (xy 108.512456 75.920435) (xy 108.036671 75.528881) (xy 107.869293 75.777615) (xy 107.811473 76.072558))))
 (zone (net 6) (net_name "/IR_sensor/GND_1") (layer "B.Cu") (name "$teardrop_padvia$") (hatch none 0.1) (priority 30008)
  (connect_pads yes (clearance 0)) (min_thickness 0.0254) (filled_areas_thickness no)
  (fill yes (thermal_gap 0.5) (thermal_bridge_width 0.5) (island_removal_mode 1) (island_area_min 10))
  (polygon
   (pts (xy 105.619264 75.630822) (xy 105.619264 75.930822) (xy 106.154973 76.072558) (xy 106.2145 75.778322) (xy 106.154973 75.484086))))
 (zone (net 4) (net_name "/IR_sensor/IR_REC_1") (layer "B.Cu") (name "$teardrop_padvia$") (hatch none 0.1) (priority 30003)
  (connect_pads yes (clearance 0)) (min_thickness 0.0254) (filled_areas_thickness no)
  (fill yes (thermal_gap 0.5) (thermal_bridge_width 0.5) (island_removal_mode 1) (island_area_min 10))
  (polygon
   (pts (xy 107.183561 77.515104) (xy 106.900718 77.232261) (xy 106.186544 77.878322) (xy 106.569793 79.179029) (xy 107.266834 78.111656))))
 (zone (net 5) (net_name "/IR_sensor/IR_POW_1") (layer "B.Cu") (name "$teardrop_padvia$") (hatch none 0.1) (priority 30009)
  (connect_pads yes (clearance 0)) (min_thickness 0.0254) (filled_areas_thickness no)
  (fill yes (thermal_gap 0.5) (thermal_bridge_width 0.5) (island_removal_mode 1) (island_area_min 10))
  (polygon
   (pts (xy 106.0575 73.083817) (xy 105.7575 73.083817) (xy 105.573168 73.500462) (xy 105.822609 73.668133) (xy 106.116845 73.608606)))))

